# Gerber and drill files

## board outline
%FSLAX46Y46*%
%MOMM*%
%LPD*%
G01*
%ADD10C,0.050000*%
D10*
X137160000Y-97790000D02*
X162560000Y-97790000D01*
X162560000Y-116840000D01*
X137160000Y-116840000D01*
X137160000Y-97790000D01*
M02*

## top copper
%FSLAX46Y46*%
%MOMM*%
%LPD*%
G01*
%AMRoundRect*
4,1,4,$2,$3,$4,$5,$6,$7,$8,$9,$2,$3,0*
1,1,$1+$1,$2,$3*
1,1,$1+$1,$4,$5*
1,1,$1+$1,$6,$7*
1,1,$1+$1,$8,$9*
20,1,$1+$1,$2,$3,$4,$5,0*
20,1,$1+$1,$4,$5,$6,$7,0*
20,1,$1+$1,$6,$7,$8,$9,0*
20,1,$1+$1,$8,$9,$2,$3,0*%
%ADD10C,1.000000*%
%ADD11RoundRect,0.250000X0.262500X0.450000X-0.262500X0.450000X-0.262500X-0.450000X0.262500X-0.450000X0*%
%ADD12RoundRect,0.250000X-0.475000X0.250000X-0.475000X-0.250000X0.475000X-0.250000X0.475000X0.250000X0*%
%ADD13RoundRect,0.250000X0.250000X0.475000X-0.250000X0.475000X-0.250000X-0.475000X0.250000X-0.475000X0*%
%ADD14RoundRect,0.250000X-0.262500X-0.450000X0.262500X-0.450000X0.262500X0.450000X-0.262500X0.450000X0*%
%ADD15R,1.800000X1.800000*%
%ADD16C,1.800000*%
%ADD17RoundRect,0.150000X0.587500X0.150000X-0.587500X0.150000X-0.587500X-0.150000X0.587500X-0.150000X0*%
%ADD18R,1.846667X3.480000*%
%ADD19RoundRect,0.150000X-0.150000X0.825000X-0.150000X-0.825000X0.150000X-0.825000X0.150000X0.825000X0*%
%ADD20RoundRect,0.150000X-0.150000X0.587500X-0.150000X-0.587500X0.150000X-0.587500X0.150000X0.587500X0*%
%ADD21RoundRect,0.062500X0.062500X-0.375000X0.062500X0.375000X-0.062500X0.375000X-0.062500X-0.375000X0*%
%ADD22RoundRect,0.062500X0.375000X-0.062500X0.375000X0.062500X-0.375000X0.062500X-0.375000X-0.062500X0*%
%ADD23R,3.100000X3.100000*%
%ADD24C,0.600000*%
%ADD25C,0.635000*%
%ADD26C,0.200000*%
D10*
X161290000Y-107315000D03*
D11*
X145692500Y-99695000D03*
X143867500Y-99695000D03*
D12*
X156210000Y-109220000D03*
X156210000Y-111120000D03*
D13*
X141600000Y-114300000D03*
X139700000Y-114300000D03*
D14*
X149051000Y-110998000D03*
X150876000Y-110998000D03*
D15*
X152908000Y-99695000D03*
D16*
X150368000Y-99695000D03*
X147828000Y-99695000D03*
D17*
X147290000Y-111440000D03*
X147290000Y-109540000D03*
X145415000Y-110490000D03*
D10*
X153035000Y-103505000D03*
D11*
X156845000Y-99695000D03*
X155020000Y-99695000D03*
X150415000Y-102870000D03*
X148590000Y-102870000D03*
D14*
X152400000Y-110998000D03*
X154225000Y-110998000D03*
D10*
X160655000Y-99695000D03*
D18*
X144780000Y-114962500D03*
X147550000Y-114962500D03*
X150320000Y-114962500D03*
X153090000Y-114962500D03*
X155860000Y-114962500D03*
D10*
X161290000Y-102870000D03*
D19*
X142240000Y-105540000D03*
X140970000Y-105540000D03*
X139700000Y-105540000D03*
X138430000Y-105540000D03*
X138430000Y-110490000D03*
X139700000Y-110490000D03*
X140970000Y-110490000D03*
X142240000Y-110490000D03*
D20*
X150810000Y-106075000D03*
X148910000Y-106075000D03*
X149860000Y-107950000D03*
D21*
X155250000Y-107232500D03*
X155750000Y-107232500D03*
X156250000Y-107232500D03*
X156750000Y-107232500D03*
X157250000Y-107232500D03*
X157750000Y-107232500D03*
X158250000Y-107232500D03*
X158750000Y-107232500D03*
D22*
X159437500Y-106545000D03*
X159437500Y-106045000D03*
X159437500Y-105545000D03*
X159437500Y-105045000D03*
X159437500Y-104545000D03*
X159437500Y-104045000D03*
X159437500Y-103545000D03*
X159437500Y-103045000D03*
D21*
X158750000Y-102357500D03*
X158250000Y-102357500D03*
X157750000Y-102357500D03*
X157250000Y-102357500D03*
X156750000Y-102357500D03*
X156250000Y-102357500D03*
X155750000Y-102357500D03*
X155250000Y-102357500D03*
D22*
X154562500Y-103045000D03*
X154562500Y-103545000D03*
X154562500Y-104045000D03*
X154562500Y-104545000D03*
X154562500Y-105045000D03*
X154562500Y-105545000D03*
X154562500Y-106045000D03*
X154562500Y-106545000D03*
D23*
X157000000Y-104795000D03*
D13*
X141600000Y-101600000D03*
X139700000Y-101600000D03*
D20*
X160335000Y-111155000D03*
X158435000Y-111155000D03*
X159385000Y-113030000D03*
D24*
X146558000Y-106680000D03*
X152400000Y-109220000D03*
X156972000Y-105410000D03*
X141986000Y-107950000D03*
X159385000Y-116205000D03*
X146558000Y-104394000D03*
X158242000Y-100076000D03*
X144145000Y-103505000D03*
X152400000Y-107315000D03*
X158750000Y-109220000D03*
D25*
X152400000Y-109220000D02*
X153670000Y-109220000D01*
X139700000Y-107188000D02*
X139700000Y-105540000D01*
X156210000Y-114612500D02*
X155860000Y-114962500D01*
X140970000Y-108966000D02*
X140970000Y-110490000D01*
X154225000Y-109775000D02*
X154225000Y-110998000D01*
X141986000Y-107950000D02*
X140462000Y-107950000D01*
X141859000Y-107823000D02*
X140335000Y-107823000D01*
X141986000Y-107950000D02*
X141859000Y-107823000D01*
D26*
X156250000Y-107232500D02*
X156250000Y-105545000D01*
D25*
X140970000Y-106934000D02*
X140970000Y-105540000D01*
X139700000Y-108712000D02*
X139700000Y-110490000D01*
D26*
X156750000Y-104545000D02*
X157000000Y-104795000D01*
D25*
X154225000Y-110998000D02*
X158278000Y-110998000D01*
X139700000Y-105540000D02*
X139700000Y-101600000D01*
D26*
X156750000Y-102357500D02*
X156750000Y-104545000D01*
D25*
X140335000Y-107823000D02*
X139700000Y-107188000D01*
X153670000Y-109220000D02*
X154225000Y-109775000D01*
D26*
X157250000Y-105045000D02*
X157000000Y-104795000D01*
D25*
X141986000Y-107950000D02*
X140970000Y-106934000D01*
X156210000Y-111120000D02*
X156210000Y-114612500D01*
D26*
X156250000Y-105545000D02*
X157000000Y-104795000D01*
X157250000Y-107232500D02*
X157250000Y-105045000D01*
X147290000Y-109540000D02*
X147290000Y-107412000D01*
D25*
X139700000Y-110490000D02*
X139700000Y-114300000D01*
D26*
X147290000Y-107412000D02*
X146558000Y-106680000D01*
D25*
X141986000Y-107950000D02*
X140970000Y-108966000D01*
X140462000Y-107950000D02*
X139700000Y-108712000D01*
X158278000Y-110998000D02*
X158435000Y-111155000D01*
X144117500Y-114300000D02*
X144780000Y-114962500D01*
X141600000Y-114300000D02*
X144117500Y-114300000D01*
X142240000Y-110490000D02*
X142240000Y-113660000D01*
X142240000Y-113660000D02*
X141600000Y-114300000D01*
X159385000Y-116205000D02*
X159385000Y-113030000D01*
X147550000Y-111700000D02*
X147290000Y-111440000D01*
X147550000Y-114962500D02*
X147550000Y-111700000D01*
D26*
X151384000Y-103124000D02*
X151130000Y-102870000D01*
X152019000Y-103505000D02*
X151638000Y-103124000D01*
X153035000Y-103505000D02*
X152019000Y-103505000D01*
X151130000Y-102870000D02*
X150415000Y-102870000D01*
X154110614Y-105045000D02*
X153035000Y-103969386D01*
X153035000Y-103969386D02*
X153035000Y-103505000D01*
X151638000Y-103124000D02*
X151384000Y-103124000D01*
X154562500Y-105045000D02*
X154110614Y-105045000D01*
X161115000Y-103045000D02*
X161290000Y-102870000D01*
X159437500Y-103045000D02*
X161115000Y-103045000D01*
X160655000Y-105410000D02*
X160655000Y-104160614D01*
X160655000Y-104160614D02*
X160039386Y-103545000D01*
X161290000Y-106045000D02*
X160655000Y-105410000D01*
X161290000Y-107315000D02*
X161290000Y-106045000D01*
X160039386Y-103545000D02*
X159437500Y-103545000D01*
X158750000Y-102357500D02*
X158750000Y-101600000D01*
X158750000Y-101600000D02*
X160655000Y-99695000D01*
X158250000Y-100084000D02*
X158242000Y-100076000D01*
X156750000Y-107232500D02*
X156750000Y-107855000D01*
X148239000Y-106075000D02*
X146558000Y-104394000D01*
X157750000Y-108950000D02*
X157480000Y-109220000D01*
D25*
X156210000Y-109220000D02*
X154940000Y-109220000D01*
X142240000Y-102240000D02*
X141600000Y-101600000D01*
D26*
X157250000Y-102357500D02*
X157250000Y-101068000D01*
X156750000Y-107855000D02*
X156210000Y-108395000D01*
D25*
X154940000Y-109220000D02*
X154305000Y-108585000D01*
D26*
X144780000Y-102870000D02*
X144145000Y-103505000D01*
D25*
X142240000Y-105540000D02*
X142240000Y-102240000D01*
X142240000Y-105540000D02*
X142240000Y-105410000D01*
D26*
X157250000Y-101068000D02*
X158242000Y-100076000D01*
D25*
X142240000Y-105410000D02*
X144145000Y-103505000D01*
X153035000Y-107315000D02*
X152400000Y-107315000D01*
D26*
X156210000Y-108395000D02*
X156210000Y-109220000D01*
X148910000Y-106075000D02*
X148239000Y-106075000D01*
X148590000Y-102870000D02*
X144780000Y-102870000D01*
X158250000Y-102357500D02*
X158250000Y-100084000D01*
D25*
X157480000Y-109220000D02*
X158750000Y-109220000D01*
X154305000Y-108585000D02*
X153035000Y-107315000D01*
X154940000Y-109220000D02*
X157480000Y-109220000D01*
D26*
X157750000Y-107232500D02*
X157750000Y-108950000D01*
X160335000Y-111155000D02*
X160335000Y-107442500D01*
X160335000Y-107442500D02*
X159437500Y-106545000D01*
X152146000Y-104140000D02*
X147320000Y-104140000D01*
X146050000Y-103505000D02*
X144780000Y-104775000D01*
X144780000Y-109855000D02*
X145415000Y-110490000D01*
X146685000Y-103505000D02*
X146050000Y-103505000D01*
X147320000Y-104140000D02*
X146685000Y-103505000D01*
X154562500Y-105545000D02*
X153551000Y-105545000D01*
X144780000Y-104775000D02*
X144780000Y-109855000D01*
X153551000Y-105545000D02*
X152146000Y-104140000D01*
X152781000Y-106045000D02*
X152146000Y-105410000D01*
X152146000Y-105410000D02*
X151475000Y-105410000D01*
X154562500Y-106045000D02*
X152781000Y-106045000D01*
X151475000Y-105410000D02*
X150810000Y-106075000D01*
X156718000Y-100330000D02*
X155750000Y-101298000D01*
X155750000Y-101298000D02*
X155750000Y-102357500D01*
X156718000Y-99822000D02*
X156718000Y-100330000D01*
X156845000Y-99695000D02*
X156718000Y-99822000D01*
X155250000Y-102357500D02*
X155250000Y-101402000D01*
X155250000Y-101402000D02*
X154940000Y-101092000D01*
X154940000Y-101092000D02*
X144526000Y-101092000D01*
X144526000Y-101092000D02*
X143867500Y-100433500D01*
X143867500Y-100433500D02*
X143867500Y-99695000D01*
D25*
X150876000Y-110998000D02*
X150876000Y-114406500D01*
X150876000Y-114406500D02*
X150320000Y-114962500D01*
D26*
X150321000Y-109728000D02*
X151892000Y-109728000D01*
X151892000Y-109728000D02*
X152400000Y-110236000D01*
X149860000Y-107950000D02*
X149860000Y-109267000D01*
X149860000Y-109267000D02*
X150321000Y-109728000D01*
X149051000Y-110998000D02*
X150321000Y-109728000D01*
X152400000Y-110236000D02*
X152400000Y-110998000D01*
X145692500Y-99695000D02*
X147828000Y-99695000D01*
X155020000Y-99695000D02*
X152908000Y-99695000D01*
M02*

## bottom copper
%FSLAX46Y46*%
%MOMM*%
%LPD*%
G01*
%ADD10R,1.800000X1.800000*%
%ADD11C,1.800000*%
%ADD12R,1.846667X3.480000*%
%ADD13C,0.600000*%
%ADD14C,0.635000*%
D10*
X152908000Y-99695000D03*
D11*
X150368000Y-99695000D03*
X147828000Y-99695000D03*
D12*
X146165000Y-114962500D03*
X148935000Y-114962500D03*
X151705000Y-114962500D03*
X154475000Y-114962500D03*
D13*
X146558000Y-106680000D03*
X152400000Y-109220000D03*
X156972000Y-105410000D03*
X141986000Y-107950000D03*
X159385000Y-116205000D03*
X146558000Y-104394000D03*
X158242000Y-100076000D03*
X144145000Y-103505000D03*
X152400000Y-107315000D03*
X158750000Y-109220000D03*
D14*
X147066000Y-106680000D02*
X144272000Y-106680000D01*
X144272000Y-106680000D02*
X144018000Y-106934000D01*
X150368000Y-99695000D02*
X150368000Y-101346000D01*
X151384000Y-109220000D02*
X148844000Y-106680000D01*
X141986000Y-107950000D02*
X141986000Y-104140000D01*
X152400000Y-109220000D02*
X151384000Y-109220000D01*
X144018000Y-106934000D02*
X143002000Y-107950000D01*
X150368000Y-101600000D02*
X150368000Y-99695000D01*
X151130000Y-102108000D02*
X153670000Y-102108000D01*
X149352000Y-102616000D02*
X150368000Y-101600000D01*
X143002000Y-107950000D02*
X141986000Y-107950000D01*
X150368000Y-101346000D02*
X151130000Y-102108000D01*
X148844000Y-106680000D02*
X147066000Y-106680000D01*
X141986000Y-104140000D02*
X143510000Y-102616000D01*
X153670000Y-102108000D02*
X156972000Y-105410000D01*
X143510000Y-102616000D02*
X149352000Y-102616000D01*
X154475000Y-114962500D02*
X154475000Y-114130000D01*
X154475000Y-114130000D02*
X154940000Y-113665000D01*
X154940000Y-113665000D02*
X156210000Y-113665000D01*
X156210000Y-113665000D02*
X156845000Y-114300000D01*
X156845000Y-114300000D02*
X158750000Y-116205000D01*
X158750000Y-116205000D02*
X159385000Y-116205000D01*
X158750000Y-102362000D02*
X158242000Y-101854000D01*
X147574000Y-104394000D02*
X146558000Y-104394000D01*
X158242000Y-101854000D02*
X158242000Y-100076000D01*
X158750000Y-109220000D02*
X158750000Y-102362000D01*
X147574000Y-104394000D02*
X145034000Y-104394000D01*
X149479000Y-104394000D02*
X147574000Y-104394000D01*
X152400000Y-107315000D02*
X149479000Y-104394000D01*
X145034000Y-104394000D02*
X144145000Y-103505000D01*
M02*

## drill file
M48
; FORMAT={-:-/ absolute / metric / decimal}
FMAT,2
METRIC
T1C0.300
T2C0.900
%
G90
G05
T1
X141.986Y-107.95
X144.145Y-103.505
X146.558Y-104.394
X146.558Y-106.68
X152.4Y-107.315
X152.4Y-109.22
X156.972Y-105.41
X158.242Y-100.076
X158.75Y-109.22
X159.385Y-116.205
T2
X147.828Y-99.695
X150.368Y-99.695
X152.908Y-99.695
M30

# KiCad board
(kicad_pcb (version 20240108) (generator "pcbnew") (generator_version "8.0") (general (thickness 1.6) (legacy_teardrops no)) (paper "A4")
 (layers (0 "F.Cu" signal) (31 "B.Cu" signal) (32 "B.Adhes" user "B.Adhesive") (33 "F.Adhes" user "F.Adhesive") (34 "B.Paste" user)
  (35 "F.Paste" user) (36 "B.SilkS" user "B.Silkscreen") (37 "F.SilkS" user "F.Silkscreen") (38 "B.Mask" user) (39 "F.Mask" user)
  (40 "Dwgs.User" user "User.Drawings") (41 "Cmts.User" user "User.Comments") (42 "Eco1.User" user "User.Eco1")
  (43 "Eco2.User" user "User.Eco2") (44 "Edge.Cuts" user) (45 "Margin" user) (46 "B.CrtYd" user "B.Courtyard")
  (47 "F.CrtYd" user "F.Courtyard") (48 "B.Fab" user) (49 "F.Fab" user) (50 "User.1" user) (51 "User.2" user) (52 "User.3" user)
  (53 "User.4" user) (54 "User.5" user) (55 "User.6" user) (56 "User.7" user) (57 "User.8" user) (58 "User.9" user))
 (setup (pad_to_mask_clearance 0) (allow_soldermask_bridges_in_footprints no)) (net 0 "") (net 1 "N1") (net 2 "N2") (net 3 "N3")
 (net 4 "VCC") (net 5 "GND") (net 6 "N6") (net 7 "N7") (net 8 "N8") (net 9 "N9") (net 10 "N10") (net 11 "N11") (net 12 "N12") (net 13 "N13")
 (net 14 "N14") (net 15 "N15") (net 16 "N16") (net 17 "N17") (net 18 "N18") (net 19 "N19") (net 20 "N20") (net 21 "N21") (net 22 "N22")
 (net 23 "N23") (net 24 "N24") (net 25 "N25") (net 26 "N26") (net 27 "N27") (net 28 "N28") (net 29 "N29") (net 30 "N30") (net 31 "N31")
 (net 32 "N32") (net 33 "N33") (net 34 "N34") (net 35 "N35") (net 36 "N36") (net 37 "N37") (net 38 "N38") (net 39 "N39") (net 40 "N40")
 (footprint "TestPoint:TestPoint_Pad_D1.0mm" (layer "F.Cu") (at 161.29 107.315)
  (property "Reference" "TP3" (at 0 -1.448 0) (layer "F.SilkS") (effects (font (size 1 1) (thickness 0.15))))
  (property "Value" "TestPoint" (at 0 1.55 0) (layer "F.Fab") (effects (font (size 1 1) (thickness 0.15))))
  (pad "1" smd circle (at 0 0) (size 1 1) (layers "F.Cu" "F.Mask") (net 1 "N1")))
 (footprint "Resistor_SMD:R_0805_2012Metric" (layer "F.Cu") (at 144.78 99.695 180)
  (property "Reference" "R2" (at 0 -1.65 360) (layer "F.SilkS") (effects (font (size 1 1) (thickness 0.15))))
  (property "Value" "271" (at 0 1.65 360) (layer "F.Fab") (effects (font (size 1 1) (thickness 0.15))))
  (pad "1" smd roundrect (at -0.9125 0 180) (size 1.025 1.4) (layers "F.Cu" "F.Paste" "F.Mask") (roundrect_rratio 0.243902) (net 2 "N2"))
  (pad "2" smd roundrect (at 0.9125 0 180) (size 1.025 1.4) (layers "F.Cu" "F.Paste" "F.Mask") (roundrect_rratio 0.243902) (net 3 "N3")))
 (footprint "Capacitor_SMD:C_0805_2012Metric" (layer "F.Cu") (at 156.21 110.17 -90)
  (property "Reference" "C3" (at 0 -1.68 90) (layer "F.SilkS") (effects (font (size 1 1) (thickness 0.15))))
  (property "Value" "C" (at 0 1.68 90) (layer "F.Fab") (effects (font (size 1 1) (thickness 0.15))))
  (pad "1" smd roundrect (at -0.95 0 270) (size 1 1.45) (layers "F.Cu" "F.Paste" "F.Mask") (roundrect_rratio 0.25) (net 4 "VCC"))
  (pad "2" smd roundrect (at 0.95 0 270) (size 1 1.45) (layers "F.Cu" "F.Paste" "F.Mask") (roundrect_rratio 0.25) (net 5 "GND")))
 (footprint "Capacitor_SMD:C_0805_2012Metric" (layer "F.Cu") (at 140.65 114.3 180)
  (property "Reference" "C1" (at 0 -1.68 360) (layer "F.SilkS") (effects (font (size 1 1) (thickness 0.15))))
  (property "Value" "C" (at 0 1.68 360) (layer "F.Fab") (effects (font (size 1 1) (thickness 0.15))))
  (pad "1" smd roundrect (at -0.95 0 180) (size 1 1.45) (layers "F.Cu" "F.Paste" "F.Mask") (roundrect_rratio 0.25) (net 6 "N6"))
  (pad "2" smd roundrect (at 0.95 0 180) (size 1 1.45) (layers "F.Cu" "F.Paste" "F.Mask") (roundrect_rratio 0.25) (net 5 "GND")))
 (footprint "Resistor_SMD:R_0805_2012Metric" (layer "F.Cu") (at 149.9635 110.998)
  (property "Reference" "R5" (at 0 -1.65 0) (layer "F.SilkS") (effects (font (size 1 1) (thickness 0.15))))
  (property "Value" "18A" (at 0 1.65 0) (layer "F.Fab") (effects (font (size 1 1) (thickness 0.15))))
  (pad "1" smd roundrect (at -0.9125 0) (size 1.025 1.4) (layers "F.Cu" "F.Paste" "F.Mask") (roundrect_rratio 0.243902) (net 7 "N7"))
  (pad "2" smd roundrect (at 0.9125 0) (size 1.025 1.4) (layers "F.Cu" "F.Paste" "F.Mask") (roundrect_rratio 0.243902) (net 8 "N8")))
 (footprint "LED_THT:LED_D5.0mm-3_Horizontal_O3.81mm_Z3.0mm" (layer "F.Cu") (at 152.908 99.695 180)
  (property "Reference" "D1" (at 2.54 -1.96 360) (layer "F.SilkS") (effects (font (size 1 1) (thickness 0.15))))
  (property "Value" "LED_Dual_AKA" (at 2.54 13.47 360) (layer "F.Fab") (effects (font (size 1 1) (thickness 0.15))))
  (pad "1" thru_hole rect (at 0 0 180) (size 1.8 1.8) (drill 0.9) (layers "*.Cu" "*.Mask") (remove_unused_layers no) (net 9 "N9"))
  (pad "2" thru_hole circle (at 2.54 0 180) (size 1.8 1.8) (drill 0.9) (layers "*.Cu" "*.Mask") (remove_unused_layers no) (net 5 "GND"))
  (pad "3" thru_hole circle (at 5.08 0 180) (size 1.8 1.8) (drill 0.9) (layers "*.Cu" "*.Mask") (remove_unused_layers no) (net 2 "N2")))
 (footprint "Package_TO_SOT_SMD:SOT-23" (layer "F.Cu") (at 146.3525 110.49 180)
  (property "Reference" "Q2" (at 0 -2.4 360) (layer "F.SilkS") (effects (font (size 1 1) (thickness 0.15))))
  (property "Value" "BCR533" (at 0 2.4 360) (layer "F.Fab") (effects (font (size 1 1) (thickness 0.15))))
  (pad "1" smd roundrect (at -0.9375 -0.95 180) (size 1.475 0.6) (layers "F.Cu" "F.Paste" "F.Mask") (roundrect_rratio 0.25) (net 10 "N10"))
  (pad "2" smd roundrect (at -0.9375 0.95 180) (size 1.475 0.6) (layers "F.Cu" "F.Paste" "F.Mask") (roundrect_rratio 0.25) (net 5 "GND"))
  (pad "3" smd roundrect (at 0.9375 0 180) (size 1.475 0.6) (layers "F.Cu" "F.Paste" "F.Mask") (roundrect_rratio 0.25) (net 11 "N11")))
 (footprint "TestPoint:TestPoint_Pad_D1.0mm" (layer "F.Cu") (at 153.035 103.505)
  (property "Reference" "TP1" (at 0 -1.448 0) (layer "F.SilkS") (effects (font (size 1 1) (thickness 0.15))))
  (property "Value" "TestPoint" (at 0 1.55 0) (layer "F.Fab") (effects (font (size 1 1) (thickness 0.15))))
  (pad "1" smd circle (at 0 0) (size 1 1) (layers "F.Cu" "F.Mask") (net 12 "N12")))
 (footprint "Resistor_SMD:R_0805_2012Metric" (layer "F.Cu") (at 155.9325 99.695 180)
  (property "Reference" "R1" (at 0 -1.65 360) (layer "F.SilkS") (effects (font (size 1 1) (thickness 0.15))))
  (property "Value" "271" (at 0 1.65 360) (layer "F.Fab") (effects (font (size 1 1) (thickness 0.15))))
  (pad "1" smd roundrect (at -0.9125 0 180) (size 1.025 1.4) (layers "F.Cu" "F.Paste" "F.Mask") (roundrect_rratio 0.243902) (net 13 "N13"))
  (pad "2" smd roundrect (at 0.9125 0 180) (size 1.025 1.4) (layers "F.Cu" "F.Paste" "F.Mask") (roundrect_rratio 0.243902) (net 9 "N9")))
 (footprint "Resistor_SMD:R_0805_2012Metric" (layer "F.Cu") (at 149.5025 102.87 180)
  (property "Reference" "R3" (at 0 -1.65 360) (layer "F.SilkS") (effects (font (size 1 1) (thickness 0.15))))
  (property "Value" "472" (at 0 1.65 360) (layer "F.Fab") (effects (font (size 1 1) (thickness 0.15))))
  (pad "1" smd roundrect (at -0.9125 0 180) (size 1.025 1.4) (layers "F.Cu" "F.Paste" "F.Mask") (roundrect_rratio 0.243902) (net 12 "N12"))
  (pad "2" smd roundrect (at 0.9125 0 180) (size 1.025 1.4) (layers "F.Cu" "F.Paste" "F.Mask") (roundrect_rratio 0.243902) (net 4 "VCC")))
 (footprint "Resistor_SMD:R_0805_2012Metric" (layer "F.Cu") (at 153.3125 110.998)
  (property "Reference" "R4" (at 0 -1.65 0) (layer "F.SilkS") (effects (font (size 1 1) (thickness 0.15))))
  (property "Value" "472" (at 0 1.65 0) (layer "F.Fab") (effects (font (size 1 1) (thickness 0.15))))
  (pad "1" smd roundrect (at -0.9125 0) (size 1.025 1.4) (layers "F.Cu" "F.Paste" "F.Mask") (roundrect_rratio 0.243902) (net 7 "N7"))
  (pad "2" smd roundrect (at 0.9125 0) (size 1.025 1.4) (layers "F.Cu" "F.Paste" "F.Mask") (roundrect_rratio 0.243902) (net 5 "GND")))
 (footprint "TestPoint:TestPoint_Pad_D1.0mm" (layer "F.Cu") (at 160.655 99.695)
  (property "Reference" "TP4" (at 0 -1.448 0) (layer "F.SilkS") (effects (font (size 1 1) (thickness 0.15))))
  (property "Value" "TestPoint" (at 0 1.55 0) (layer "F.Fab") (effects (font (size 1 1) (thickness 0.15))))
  (pad "1" smd circle (at 0 0) (size 1 1) (layers "F.Cu" "F.Mask") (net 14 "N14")))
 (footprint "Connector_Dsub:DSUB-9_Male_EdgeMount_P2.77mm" (layer "F.Cu") (at 150.32 114.9625)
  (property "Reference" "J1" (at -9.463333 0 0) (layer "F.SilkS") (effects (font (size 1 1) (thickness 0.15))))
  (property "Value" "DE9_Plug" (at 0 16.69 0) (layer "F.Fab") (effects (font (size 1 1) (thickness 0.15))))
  (pad "1" smd rect (at -5.54 0) (size 1.846667 3.48) (layers "F.Cu" "F.Paste" "F.Mask") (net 6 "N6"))
  (pad "2" smd rect (at -2.77 0) (size 1.846667 3.48) (layers "F.Cu" "F.Paste" "F.Mask") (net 10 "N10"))
  (pad "3" smd rect (at 0 0) (size 1.846667 3.48) (layers "F.Cu" "F.Paste" "F.Mask") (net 8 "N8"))
  (pad "4" smd rect (at 2.77 0) (size 1.846667 3.48) (layers "F.Cu" "F.Paste" "F.Mask") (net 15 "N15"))
  (pad "5" smd rect (at 5.54 0) (size 1.846667 3.48) (layers "F.Cu" "F.Paste" "F.Mask") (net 5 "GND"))
  (pad "6" smd rect (at -4.155 0) (size 1.846667 3.48) (layers "B.Cu" "B.Paste" "B.Mask") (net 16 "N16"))
  (pad "7" smd rect (at -1.385 0) (size 1.846667 3.48) (layers "B.Cu" "B.Paste" "B.Mask") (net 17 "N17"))
  (pad "8" smd rect (at 1.385 0) (size 1.846667 3.48) (layers "B.Cu" "B.Paste" "B.Mask") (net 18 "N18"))
  (pad "9" smd rect (at 4.155 0) (size 1.846667 3.48) (layers "B.Cu" "B.Paste" "B.Mask") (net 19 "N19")))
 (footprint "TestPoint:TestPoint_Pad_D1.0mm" (layer "F.Cu") (at 161.29 102.87)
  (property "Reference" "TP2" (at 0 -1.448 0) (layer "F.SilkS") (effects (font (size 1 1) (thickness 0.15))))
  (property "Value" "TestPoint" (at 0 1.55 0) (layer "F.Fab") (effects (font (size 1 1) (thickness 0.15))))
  (pad "1" smd circle (at 0 0) (size 1 1) (layers "F.Cu" "F.Mask") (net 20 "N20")))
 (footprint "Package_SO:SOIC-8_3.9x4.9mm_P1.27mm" (layer "F.Cu") (at 140.335 108.015 -90)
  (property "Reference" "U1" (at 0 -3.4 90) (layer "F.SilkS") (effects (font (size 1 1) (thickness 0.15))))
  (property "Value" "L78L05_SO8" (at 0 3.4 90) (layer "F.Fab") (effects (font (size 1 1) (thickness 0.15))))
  (pad "1" smd roundrect (at -2.475 -1.905 270) (size 1.95 0.6) (layers "F.Cu" "F.Paste" "F.Mask") (roundrect_rratio 0.25) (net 4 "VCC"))
  (pad "2" smd roundrect (at -2.475 -0.635 270) (size 1.95 0.6) (layers "F.Cu" "F.Paste" "F.Mask") (roundrect_rratio 0.25) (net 5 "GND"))
  (pad "3" smd roundrect (at -2.475 0.635 270) (size 1.95 0.6) (layers "F.Cu" "F.Paste" "F.Mask") (roundrect_rratio 0.25) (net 5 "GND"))
  (pad "4" smd roundrect (at -2.475 1.905 270) (size 1.95 0.6) (layers "F.Cu" "F.Paste" "F.Mask") (roundrect_rratio 0.25) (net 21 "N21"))
  (pad "5" smd roundrect (at 2.475 1.905 270) (size 1.95 0.6) (layers "F.Cu" "F.Paste" "F.Mask") (roundrect_rratio 0.25) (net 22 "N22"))
  (pad "6" smd roundrect (at 2.475 0.635 270) (size 1.95 0.6) (layers "F.Cu" "F.Paste" "F.Mask") (roundrect_rratio 0.25) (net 5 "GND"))
  (pad "7" smd roundrect (at 2.475 -0.635 270) (size 1.95 0.6) (layers "F.Cu" "F.Paste" "F.Mask") (roundrect_rratio 0.25) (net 5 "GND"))
  (pad "8" smd roundrect (at 2.475 -1.905 270) (size 1.95 0.6) (layers "F.Cu" "F.Paste" "F.Mask") (roundrect_rratio 0.25) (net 6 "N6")))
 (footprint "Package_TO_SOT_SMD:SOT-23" (layer "F.Cu") (at 149.86 107.0125 -90)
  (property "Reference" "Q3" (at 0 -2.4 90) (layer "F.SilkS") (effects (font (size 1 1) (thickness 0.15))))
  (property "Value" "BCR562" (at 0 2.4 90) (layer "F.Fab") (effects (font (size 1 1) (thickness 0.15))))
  (pad "1" smd roundrect (at -0.9375 -0.95 270) (size 1.475 0.6) (layers "F.Cu" "F.Paste" "F.Mask") (roundrect_rratio 0.25) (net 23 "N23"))
  (pad "2" smd roundrect (at -0.9375 0.95 270) (size 1.475 0.6) (layers "F.Cu" "F.Paste" "F.Mask") (roundrect_rratio 0.25) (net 4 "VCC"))
  (pad "3" smd roundrect (at 0.9375 0 270) (size 1.475 0.6) (layers "F.Cu" "F.Paste" "F.Mask") (roundrect_rratio 0.25) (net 7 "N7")))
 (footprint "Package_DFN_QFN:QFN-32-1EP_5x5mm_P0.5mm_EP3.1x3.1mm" (layer "F.Cu") (at 157 104.795 90)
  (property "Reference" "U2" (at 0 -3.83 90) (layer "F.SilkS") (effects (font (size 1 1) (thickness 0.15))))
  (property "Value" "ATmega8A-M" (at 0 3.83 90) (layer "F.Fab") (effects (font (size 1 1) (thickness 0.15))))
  (pad "" smd roundrect (at -1.03 -1.03 90) (size 0.83 0.83) (layers "F.Paste") (roundrect_rratio 0.25))
  (pad "" smd roundrect (at -1.03 0 90) (size 0.83 0.83) (layers "F.Paste") (roundrect_rratio 0.25))
  (pad "" smd roundrect (at -1.03 1.03 90) (size 0.83 0.83) (layers "F.Paste") (roundrect_rratio 0.25))
  (pad "" smd roundrect (at 0 -1.03 90) (size 0.83 0.83) (layers "F.Paste") (roundrect_rratio 0.25))
  (pad "" smd roundrect (at 0 0 90) (size 0.83 0.83) (layers "F.Paste") (roundrect_rratio 0.25))
  (pad "" smd roundrect (at 0 1.03 90) (size 0.83 0.83) (layers "F.Paste") (roundrect_rratio 0.25))
  (pad "" smd roundrect (at 1.03 -1.03 90) (size 0.83 0.83) (layers "F.Paste") (roundrect_rratio 0.25))
  (pad "" smd roundrect (at 1.03 0 90) (size 0.83 0.83) (layers "F.Paste") (roundrect_rratio 0.25))
  (pad "" smd roundrect (at 1.03 1.03 90) (size 0.83 0.83) (layers "F.Paste") (roundrect_rratio 0.25))
  (pad "1" smd roundrect (at -2.4375 -1.75 90) (size 0.875 0.25) (layers "F.Cu" "F.Paste" "F.Mask") (roundrect_rratio 0.25) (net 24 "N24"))
  (pad "2" smd roundrect (at -2.4375 -1.25 90) (size 0.875 0.25) (layers "F.Cu" "F.Paste" "F.Mask") (roundrect_rratio 0.25) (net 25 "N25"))
  (pad "3" smd roundrect (at -2.4375 -0.75 90) (size 0.875 0.25) (layers "F.Cu" "F.Paste" "F.Mask") (roundrect_rratio 0.25) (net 5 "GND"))
  (pad "4" smd roundrect (at -2.4375 -0.25 90) (size 0.875 0.25) (layers "F.Cu" "F.Paste" "F.Mask") (roundrect_rratio 0.25) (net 4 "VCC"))
  (pad "5" smd roundrect (at -2.4375 0.25 90) (size 0.875 0.25) (layers "F.Cu" "F.Paste" "F.Mask") (roundrect_rratio 0.25) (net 5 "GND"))
  (pad "6" smd roundrect (at -2.4375 0.75 90) (size 0.875 0.25) (layers "F.Cu" "F.Paste" "F.Mask") (roundrect_rratio 0.25) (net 4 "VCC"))
  (pad "7" smd roundrect (at -2.4375 1.25 90) (size 0.875 0.25) (layers "F.Cu" "F.Paste" "F.Mask") (roundrect_rratio 0.25) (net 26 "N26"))
  (pad "8" smd roundrect (at -2.4375 1.75 90) (size 0.875 0.25) (layers "F.Cu" "F.Paste" "F.Mask") (roundrect_rratio 0.25) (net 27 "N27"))
  (pad "9" smd roundrect (at -1.75 2.4375 90) (size 0.25 0.875) (layers "F.Cu" "F.Paste" "F.Mask") (roundrect_rratio 0.25) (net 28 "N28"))
  (pad "10" smd roundrect (at -1.25 2.4375 90) (size 0.25 0.875) (layers "F.Cu" "F.Paste" "F.Mask") (roundrect_rratio 0.25) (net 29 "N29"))
  (pad "11" smd roundrect (at -0.75 2.4375 90) (size 0.25 0.875) (layers "F.Cu" "F.Paste" "F.Mask") (roundrect_rratio 0.25) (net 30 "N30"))
  (pad "12" smd roundrect (at -0.25 2.4375 90) (size 0.25 0.875) (layers "F.Cu" "F.Paste" "F.Mask") (roundrect_rratio 0.25) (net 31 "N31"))
  (pad "13" smd roundrect (at 0.25 2.4375 90) (size 0.25 0.875) (layers "F.Cu" "F.Paste" "F.Mask") (roundrect_rratio 0.25) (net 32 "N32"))
  (pad "14" smd roundrect (at 0.75 2.4375 90) (size 0.25 0.875) (layers "F.Cu" "F.Paste" "F.Mask") (roundrect_rratio 0.25) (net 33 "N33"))
  (pad "15" smd roundrect (at 1.25 2.4375 90) (size 0.25 0.875) (layers "F.Cu" "F.Paste" "F.Mask") (roundrect_rratio 0.25) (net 1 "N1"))
  (pad "16" smd roundrect (at 1.75 2.4375 90) (size 0.25 0.875) (layers "F.Cu" "F.Paste" "F.Mask") (roundrect_rratio 0.25) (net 20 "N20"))
  (pad "17" smd roundrect (at 2.4375 1.75 90) (size 0.875 0.25) (layers "F.Cu" "F.Paste" "F.Mask") (roundrect_rratio 0.25) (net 14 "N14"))
  (pad "18" smd roundrect (at 2.4375 1.25 90) (size 0.875 0.25) (layers "F.Cu" "F.Paste" "F.Mask") (roundrect_rratio 0.25) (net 4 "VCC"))
  (pad "19" smd roundrect (at 2.4375 0.75 90) (size 0.875 0.25) (layers "F.Cu" "F.Paste" "F.Mask") (roundrect_rratio 0.25) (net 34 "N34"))
  (pad "20" smd roundrect (at 2.4375 0.25 90) (size 0.875 0.25) (layers "F.Cu" "F.Paste" "F.Mask") (roundrect_rratio 0.25) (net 4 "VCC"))
  (pad "21" smd roundrect (at 2.4375 -0.25 90) (size 0.875 0.25) (layers "F.Cu" "F.Paste" "F.Mask") (roundrect_rratio 0.25) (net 5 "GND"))
  (pad "22" smd roundrect (at 2.4375 -0.75 90) (size 0.875 0.25) (layers "F.Cu" "F.Paste" "F.Mask") (roundrect_rratio 0.25) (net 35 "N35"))
  (pad "23" smd roundrect (at 2.4375 -1.25 90) (size 0.875 0.25) (layers "F.Cu" "F.Paste" "F.Mask") (roundrect_rratio 0.25) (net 13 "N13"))
  (pad "24" smd roundrect (at 2.4375 -1.75 90) (size 0.875 0.25) (layers "F.Cu" "F.Paste" "F.Mask") (roundrect_rratio 0.25) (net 3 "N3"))
  (pad "25" smd roundrect (at 1.75 -2.4375 90) (size 0.25 0.875) (layers "F.Cu" "F.Paste" "F.Mask") (roundrect_rratio 0.25) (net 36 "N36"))
  (pad "26" smd roundrect (at 1.25 -2.4375 90) (size 0.25 0.875) (layers "F.Cu" "F.Paste" "F.Mask") (roundrect_rratio 0.25) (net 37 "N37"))
  (pad "27" smd roundrect (at 0.75 -2.4375 90) (size 0.25 0.875) (layers "F.Cu" "F.Paste" "F.Mask") (roundrect_rratio 0.25) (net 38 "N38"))
  (pad "28" smd roundrect (at 0.25 -2.4375 90) (size 0.25 0.875) (layers "F.Cu" "F.Paste" "F.Mask") (roundrect_rratio 0.25) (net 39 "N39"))
  (pad "29" smd roundrect (at -0.25 -2.4375 90) (size 0.25 0.875) (layers "F.Cu" "F.Paste" "F.Mask") (roundrect_rratio 0.25) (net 12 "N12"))
  (pad "30" smd roundrect (at -0.75 -2.4375 90) (size 0.25 0.875) (layers "F.Cu" "F.Paste" "F.Mask") (roundrect_rratio 0.25) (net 11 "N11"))
  (pad "31" smd roundrect (at -1.25 -2.4375 90) (size 0.25 0.875) (layers "F.Cu" "F.Paste" "F.Mask") (roundrect_rratio 0.25) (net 23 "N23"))
  (pad "32" smd roundrect (at -1.75 -2.4375 90) (size 0.25 0.875) (layers "F.Cu" "F.Paste" "F.Mask") (roundrect_rratio 0.25) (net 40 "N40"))
  (pad "33" smd rect (at 0 0 90) (size 3.1 3.1) (layers "F.Cu" "F.Mask") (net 5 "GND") (zone_connect 2)))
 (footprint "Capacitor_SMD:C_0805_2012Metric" (layer "F.Cu") (at 140.65 101.6 180)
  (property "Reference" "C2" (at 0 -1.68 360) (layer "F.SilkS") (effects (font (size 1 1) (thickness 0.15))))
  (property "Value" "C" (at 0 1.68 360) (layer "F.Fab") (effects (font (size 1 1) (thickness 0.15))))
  (pad "1" smd roundrect (at -0.95 0 180) (size 1 1.45) (layers "F.Cu" "F.Paste" "F.Mask") (roundrect_rratio 0.25) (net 4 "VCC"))
  (pad "2" smd roundrect (at 0.95 0 180) (size 1 1.45) (layers "F.Cu" "F.Paste" "F.Mask") (roundrect_rratio 0.25) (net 5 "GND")))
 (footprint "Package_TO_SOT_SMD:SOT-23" (layer "F.Cu") (at 159.385 112.0925 -90)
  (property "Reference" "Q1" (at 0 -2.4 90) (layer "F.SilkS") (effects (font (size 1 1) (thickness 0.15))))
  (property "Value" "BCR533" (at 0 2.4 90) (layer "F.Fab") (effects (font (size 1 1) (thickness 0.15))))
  (pad "1" smd roundrect (at -0.9375 -0.95 270) (size 1.475 0.6) (layers "F.Cu" "F.Paste" "F.Mask") (roundrect_rratio 0.25) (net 28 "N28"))
  (pad "2" smd roundrect (at -0.9375 0.95 270) (size 1.475 0.6) (layers "F.Cu" "F.Paste" "F.Mask") (roundrect_rratio 0.25) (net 5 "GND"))
  (pad "3" smd roundrect (at 0.9375 0 270) (size 1.475 0.6) (layers "F.Cu" "F.Paste" "F.Mask") (roundrect_rratio 0.25) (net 19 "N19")))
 (gr_rect (start 137.16 97.79) (end 162.56 116.84) (stroke (width 0.05) (type default)) (fill none) (layer "Edge.Cuts"))
 (segment (start 152.4 109.22) (end 153.67 109.22) (width 0.635) (layer "F.Cu") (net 5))
 (segment (start 139.7 107.188) (end 139.7 105.54) (width 0.635) (layer "F.Cu") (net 5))
 (segment (start 156.21 114.6125) (end 155.86 114.9625) (width 0.635) (layer "F.Cu") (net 5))
 (segment (start 140.97 108.966) (end 140.97 110.49) (width 0.635) (layer "F.Cu") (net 5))
 (segment (start 154.225 109.775) (end 154.225 110.998) (width 0.635) (layer "F.Cu") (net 5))
 (segment (start 141.986 107.95) (end 140.462 107.95) (width 0.635) (layer "F.Cu") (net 5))
 (segment (start 141.859 107.823) (end 140.335 107.823) (width 0.635) (layer "F.Cu") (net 5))
 (segment (start 141.986 107.95) (end 141.859 107.823) (width 0.635) (layer "F.Cu") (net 5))
 (segment (start 156.25 107.2325) (end 156.25 105.545) (width 0.2) (layer "F.Cu") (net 5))
 (segment (start 140.97 106.934) (end 140.97 105.54) (width 0.635) (layer "F.Cu") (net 5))
 (segment (start 139.7 108.712) (end 139.7 110.49) (width 0.635) (layer "F.Cu") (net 5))
 (segment (start 156.75 104.545) (end 157 104.795) (width 0.2) (layer "F.Cu") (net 5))
 (segment (start 154.225 110.998) (end 158.278 110.998) (width 0.635) (layer "F.Cu") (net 5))
 (segment (start 139.7 105.54) (end 139.7 101.6) (width 0.635) (layer "F.Cu") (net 5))
 (segment (start 156.75 102.3575) (end 156.75 104.545) (width 0.2) (layer "F.Cu") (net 5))
 (segment (start 140.335 107.823) (end 139.7 107.188) (width 0.635) (layer "F.Cu") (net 5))
 (segment (start 153.67 109.22) (end 154.225 109.775) (width 0.635) (layer "F.Cu") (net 5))
 (segment (start 157.25 105.045) (end 157 104.795) (width 0.2) (layer "F.Cu") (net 5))
 (segment (start 141.986 107.95) (end 140.97 106.934) (width 0.635) (layer "F.Cu") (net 5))
 (segment (start 156.21 111.12) (end 156.21 114.6125) (width 0.635) (layer "F.Cu") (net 5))
 (segment (start 156.25 105.545) (end 157 104.795) (width 0.2) (layer "F.Cu") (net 5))
 (segment (start 157.25 107.2325) (end 157.25 105.045) (width 0.2) (layer "F.Cu") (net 5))
 (segment (start 147.29 109.54) (end 147.29 107.412) (width 0.2) (layer "F.Cu") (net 5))
 (segment (start 139.7 110.49) (end 139.7 114.3) (width 0.635) (layer "F.Cu") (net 5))
 (segment (start 147.29 107.412) (end 146.558 106.68) (width 0.2) (layer "F.Cu") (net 5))
 (segment (start 141.986 107.95) (end 140.97 108.966) (width 0.635) (layer "F.Cu") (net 5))
 (segment (start 140.462 107.95) (end 139.7 108.712) (width 0.635) (layer "F.Cu") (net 5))
 (segment (start 158.278 110.998) (end 158.435 111.155) (width 0.635) (layer "F.Cu") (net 5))
 (via (at 146.558 106.68) (size 0.6) (drill 0.3) (layers "F.Cu" "B.Cu") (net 5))
 (via (at 152.4 109.22) (size 0.6) (drill 0.3) (layers "F.Cu" "B.Cu") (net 5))
 (via (at 156.972 105.41) (size 0.6) (drill 0.3) (layers "F.Cu" "B.Cu") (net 5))
 (via (at 141.986 107.95) (size 0.6) (drill 0.3) (layers "F.Cu" "B.Cu") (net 5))
 (segment (start 147.066 106.68) (end 144.272 106.68) (width 0.635) (layer "B.Cu") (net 5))
 (segment (start 144.272 106.68) (end 144.018 106.934) (width 0.635) (layer "B.Cu") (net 5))
 (segment (start 150.368 99.695) (end 150.368 101.346) (width 0.635) (layer "B.Cu") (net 5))
 (segment (start 151.384 109.22) (end 148.844 106.68) (width 0.635) (layer "B.Cu") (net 5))
 (segment (start 141.986 107.95) (end 141.986 104.14) (width 0.635) (layer "B.Cu") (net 5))
 (segment (start 152.4 109.22) (end 151.384 109.22) (width 0.635) (layer "B.Cu") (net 5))
 (segment (start 144.018 106.934) (end 143.002 107.95) (width 0.635) (layer "B.Cu") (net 5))
 (segment (start 150.368 101.6) (end 150.368 99.695) (width 0.635) (layer "B.Cu") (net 5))
 (segment (start 151.13 102.108) (end 153.67 102.108) (width 0.635) (layer "B.Cu") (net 5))
 (segment (start 149.352 102.616) (end 150.368 101.6) (width 0.635) (layer "B.Cu") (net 5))
 (segment (start 143.002 107.95) (end 141.986 107.95) (width 0.635) (layer "B.Cu") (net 5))
 (segment (start 150.368 101.346) (end 151.13 102.108) (width 0.635) (layer "B.Cu") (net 5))
 (segment (start 148.844 106.68) (end 147.066 106.68) (width 0.635) (layer "B.Cu") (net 5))
 (segment (start 141.986 104.14) (end 143.51 102.616) (width 0.635) (layer "B.Cu") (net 5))
 (segment (start 153.67 102.108) (end 156.972 105.41) (width 0.635) (layer "B.Cu") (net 5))
 (segment (start 143.51 102.616) (end 149.352 102.616) (width 0.635) (layer "B.Cu") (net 5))
 (segment (start 144.1175 114.3) (end 144.78 114.9625) (width 0.635) (layer "F.Cu") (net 6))
 (segment (start 141.6 114.3) (end 144.1175 114.3) (width 0.635) (layer "F.Cu") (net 6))
 (segment (start 142.24 110.49) (end 142.24 113.66) (width 0.635) (layer "F.Cu") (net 6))
 (segment (start 142.24 113.66) (end 141.6 114.3) (width 0.635) (layer "F.Cu") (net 6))
 (segment (start 159.385 116.205) (end 159.385 113.03) (width 0.635) (layer "F.Cu") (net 19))
 (via (at 159.385 116.205) (size 0.6) (drill 0.3) (layers "F.Cu" "B.Cu") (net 19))
 (segment (start 154.475 114.9625) (end 154.475 114.13) (width 0.635) (layer "B.Cu") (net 19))
 (segment (start 154.475 114.13) (end 154.94 113.665) (width 0.635) (layer "B.Cu") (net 19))
 (segment (start 154.94 113.665) (end 156.21 113.665) (width 0.635) (layer "B.Cu") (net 19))
 (segment (start 156.21 113.665) (end 156.845 114.3) (width 0.635) (layer "B.Cu") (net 19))
 (segment (start 156.845 114.3) (end 158.75 116.205) (width 0.635) (layer "B.Cu") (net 19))
 (segment (start 158.75 116.205) (end 159.385 116.205) (width 0.635) (layer "B.Cu") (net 19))
 (segment (start 147.55 111.7) (end 147.29 111.44) (width 0.635) (layer "F.Cu") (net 10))
 (segment (start 147.55 114.9625) (end 147.55 111.7) (width 0.635) (layer "F.Cu") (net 10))
 (segment (start 151.384 103.124) (end 151.13 102.87) (width 0.2) (layer "F.Cu") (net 12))
 (segment (start 152.019 103.505) (end 151.638 103.124) (width 0.2) (layer "F.Cu") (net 12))
 (segment (start 153.035 103.505) (end 152.019 103.505) (width 0.2) (layer "F.Cu") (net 12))
 (segment (start 151.13 102.87) (end 150.415 102.87) (width 0.2) (layer "F.Cu") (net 12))
 (segment (start 154.110614 105.045) (end 153.035 103.969386) (width 0.2) (layer "F.Cu") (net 12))
 (segment (start 153.035 103.969386) (end 153.035 103.505) (width 0.2) (layer "F.Cu") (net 12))
 (segment (start 151.638 103.124) (end 151.384 103.124) (width 0.2) (layer "F.Cu") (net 12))
 (segment (start 154.5625 105.045) (end 154.110614 105.045) (width 0.2) (layer "F.Cu") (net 12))
 (segment (start 161.115 103.045) (end 161.29 102.87) (width 0.2) (layer "F.Cu") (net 20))
 (segment (start 159.4375 103.045) (end 161.115 103.045) (width 0.2) (layer "F.Cu") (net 20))
 (segment (start 160.655 105.41) (end 160.655 104.160614) (width 0.2) (layer "F.Cu") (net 1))
 (segment (start 160.655 104.160614) (end 160.039386 103.545) (width 0.2) (layer "F.Cu") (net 1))
 (segment (start 161.29 106.045) (end 160.655 105.41) (width 0.2) (layer "F.Cu") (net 1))
 (segment (start 161.29 107.315) (end 161.29 106.045) (width 0.2) (layer "F.Cu") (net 1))
 (segment (start 160.039386 103.545) (end 159.4375 103.545) (width 0.2) (layer "F.Cu") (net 1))
 (segment (start 158.75 102.3575) (end 158.75 101.6) (width 0.2) (layer "F.Cu") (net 14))
 (segment (start 158.75 101.6) (end 160.655 99.695) (width 0.2) (layer "F.Cu") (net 14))
 (segment (start 158.25 100.084) (end 158.242 100.076) (width 0.2) (layer "F.Cu") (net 4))
 (segment (start 156.75 107.2325) (end 156.75 107.855) (width 0.2) (layer "F.Cu") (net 4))
 (segment (start 148.239 106.075) (end 146.558 104.394) (width 0.2) (layer "F.Cu") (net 4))
 (segment (start 157.75 108.95) (end 157.48 109.22) (width 0.2) (layer "F.Cu") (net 4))
 (segment (start 156.21 109.22) (end 154.94 109.22) (width 0.635) (layer "F.Cu") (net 4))
 (segment (start 142.24 102.24) (end 141.6 101.6) (width 0.635) (layer "F.Cu") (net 4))
 (segment (start 157.25 102.3575) (end 157.25 101.068) (width 0.2) (layer "F.Cu") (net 4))
 (segment (start 156.75 107.855) (end 156.21 108.395) (width 0.2) (layer "F.Cu") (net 4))
 (segment (start 154.94 109.22) (end 154.305 108.585) (width 0.635) (layer "F.Cu") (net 4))
 (segment (start 144.78 102.87) (end 144.145 103.505) (width 0.2) (layer "F.Cu") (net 4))
 (segment (start 142.24 105.54) (end 142.24 102.24) (width 0.635) (layer "F.Cu") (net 4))
 (segment (start 142.24 105.54) (end 142.24 105.41) (width 0.635) (layer "F.Cu") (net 4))
 (segment (start 157.25 101.068) (end 158.242 100.076) (width 0.2) (layer "F.Cu") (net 4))
 (segment (start 142.24 105.41) (end 144.145 103.505) (width 0.635) (layer "F.Cu") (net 4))
 (segment (start 153.035 107.315) (end 152.4 107.315) (width 0.635) (layer "F.Cu") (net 4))
 (segment (start 156.21 108.395) (end 156.21 109.22) (width 0.2) (layer "F.Cu") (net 4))
 (segment (start 148.91 106.075) (end 148.239 106.075) (width 0.2) (layer "F.Cu") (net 4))
 (segment (start 148.59 102.87) (end 144.78 102.87) (width 0.2) (layer "F.Cu") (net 4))
 (segment (start 158.25 102.3575) (end 158.25 100.084) (width 0.2) (layer "F.Cu") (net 4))
 (segment (start 157.48 109.22) (end 158.75 109.22) (width 0.635) (layer "F.Cu") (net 4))
 (segment (start 154.305 108.585) (end 153.035 107.315) (width 0.635) (layer "F.Cu") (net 4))
 (segment (start 154.94 109.22) (end 157.48 109.22) (width 0.635) (layer "F.Cu") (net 4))
 (segment (start 157.75 107.2325) (end 157.75 108.95) (width 0.2) (layer "F.Cu") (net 4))
 (via (at 146.558 104.394) (size 0.6) (drill 0.3) (layers "F.Cu" "B.Cu") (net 4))
 (via (at 158.242 100.076) (size 0.6) (drill 0.3) (layers "F.Cu" "B.Cu") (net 4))
 (via (at 144.145 103.505) (size 0.6) (drill 0.3) (layers "F.Cu" "B.Cu") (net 4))
 (via (at 152.4 107.315) (size 0.6) (drill 0.3) (layers "F.Cu" "B.Cu") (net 4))
 (via (at 158.75 109.22) (size 0.6) (drill 0.3) (layers "F.Cu" "B.Cu") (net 4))
 (segment (start 158.75 102.362) (end 158.242 101.854) (width 0.635) (layer "B.Cu") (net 4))
 (segment (start 147.574 104.394) (end 146.558 104.394) (width 0.635) (layer "B.Cu") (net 4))
 (segment (start 158.242 101.854) (end 158.242 100.076) (width 0.635) (layer "B.Cu") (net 4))
 (segment (start 158.75 109.22) (end 158.75 102.362) (width 0.635) (layer "B.Cu") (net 4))
 (segment (start 147.574 104.394) (end 145.034 104.394) (width 0.635) (layer "B.Cu") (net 4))
 (segment (start 149.479 104.394) (end 147.574 104.394) (width 0.635) (layer "B.Cu") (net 4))
 (segment (start 152.4 107.315) (end 149.479 104.394) (width 0.635) (layer "B.Cu") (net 4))
 (segment (start 145.034 104.394) (end 144.145 103.505) (width 0.635) (layer "B.Cu") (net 4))
 (segment (start 160.335 111.155) (end 160.335 107.4425) (width 0.2) (layer "F.Cu") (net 28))
 (segment (start 160.335 107.4425) (end 159.4375 106.545) (width 0.2) (layer "F.Cu") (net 28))
 (segment (start 152.146 104.14) (end 147.32 104.14) (width 0.2) (layer "F.Cu") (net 11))
 (segment (start 146.05 103.505) (end 144.78 104.775) (width 0.2) (layer "F.Cu") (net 11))
 (segment (start 144.78 109.855) (end 145.415 110.49) (width 0.2) (layer "F.Cu") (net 11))
 (segment (start 146.685 103.505) (end 146.05 103.505) (width 0.2) (layer "F.Cu") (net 11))
 (segment (start 147.32 104.14) (end 146.685 103.505) (width 0.2) (layer "F.Cu") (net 11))
 (segment (start 154.5625 105.545) (end 153.551 105.545) (width 0.2) (layer "F.Cu") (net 11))
 (segment (start 144.78 104.775) (end 144.78 109.855) (width 0.2) (layer "F.Cu") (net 11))
 (segment (start 153.551 105.545) (end 152.146 104.14) (width 0.2) (layer "F.Cu") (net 11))
 (segment (start 152.781 106.045) (end 152.146 105.41) (width 0.2) (layer "F.Cu") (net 23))
 (segment (start 152.146 105.41) (end 151.475 105.41) (width 0.2) (layer "F.Cu") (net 23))
 (segment (start 154.5625 106.045) (end 152.781 106.045) (width 0.2) (layer "F.Cu") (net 23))
 (segment (start 151.475 105.41) (end 150.81 106.075) (width 0.2) (layer "F.Cu") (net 23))
 (segment (start 156.718 100.33) (end 155.75 101.298) (width 0.2) (layer "F.Cu") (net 13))
 (segment (start 155.75 101.298) (end 155.75 102.3575) (width 0.2) (layer "F.Cu") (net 13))
 (segment (start 156.718 99.822) (end 156.718 100.33) (width 0.2) (layer "F.Cu") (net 13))
 (segment (start 156.845 99.695) (end 156.718 99.822) (width 0.2) (layer "F.Cu") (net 13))
 (segment (start 155.25 102.3575) (end 155.25 101.402) (width 0.2) (layer "F.Cu") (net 3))
 (segment (start 155.25 101.402) (end 154.94 101.092) (width 0.2) (layer "F.Cu") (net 3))
 (segment (start 154.94 101.092) (end 144.526 101.092) (width 0.2) (layer "F.Cu") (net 3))
 (segment (start 144.526 101.092) (end 143.8675 100.4335) (width 0.2) (layer "F.Cu") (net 3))
 (segment (start 143.8675 100.4335) (end 143.8675 99.695) (width 0.2) (layer "F.Cu") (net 3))
 (segment (start 150.876 110.998) (end 150.876 114.4065) (width 0.635) (layer "F.Cu") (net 8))
 (segment (start 150.876 114.4065) (end 150.32 114.9625) (width 0.635) (layer "F.Cu") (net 8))
 (segment (start 150.321 109.728) (end 151.892 109.728) (width 0.2) (layer "F.Cu") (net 7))
 (segment (start 151.892 109.728) (end 152.4 110.236) (width 0.2) (layer "F.Cu") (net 7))
 (segment (start 149.86 107.95) (end 149.86 109.267) (width 0.2) (layer "F.Cu") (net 7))
 (segment (start 149.86 109.267) (end 150.321 109.728) (width 0.2) (layer "F.Cu") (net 7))
 (segment (start 149.051 110.998) (end 150.321 109.728) (width 0.2) (layer "F.Cu") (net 7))
 (segment (start 152.4 110.236) (end 152.4 110.998) (width 0.2) (layer "F.Cu") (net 7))
 (segment (start 145.6925 99.695) (end 147.828 99.695) (width 0.2) (layer "F.Cu") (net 2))
 (segment (start 155.02 99.695) (end 152.908 99.695) (width 0.2) (layer "F.Cu") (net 9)))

